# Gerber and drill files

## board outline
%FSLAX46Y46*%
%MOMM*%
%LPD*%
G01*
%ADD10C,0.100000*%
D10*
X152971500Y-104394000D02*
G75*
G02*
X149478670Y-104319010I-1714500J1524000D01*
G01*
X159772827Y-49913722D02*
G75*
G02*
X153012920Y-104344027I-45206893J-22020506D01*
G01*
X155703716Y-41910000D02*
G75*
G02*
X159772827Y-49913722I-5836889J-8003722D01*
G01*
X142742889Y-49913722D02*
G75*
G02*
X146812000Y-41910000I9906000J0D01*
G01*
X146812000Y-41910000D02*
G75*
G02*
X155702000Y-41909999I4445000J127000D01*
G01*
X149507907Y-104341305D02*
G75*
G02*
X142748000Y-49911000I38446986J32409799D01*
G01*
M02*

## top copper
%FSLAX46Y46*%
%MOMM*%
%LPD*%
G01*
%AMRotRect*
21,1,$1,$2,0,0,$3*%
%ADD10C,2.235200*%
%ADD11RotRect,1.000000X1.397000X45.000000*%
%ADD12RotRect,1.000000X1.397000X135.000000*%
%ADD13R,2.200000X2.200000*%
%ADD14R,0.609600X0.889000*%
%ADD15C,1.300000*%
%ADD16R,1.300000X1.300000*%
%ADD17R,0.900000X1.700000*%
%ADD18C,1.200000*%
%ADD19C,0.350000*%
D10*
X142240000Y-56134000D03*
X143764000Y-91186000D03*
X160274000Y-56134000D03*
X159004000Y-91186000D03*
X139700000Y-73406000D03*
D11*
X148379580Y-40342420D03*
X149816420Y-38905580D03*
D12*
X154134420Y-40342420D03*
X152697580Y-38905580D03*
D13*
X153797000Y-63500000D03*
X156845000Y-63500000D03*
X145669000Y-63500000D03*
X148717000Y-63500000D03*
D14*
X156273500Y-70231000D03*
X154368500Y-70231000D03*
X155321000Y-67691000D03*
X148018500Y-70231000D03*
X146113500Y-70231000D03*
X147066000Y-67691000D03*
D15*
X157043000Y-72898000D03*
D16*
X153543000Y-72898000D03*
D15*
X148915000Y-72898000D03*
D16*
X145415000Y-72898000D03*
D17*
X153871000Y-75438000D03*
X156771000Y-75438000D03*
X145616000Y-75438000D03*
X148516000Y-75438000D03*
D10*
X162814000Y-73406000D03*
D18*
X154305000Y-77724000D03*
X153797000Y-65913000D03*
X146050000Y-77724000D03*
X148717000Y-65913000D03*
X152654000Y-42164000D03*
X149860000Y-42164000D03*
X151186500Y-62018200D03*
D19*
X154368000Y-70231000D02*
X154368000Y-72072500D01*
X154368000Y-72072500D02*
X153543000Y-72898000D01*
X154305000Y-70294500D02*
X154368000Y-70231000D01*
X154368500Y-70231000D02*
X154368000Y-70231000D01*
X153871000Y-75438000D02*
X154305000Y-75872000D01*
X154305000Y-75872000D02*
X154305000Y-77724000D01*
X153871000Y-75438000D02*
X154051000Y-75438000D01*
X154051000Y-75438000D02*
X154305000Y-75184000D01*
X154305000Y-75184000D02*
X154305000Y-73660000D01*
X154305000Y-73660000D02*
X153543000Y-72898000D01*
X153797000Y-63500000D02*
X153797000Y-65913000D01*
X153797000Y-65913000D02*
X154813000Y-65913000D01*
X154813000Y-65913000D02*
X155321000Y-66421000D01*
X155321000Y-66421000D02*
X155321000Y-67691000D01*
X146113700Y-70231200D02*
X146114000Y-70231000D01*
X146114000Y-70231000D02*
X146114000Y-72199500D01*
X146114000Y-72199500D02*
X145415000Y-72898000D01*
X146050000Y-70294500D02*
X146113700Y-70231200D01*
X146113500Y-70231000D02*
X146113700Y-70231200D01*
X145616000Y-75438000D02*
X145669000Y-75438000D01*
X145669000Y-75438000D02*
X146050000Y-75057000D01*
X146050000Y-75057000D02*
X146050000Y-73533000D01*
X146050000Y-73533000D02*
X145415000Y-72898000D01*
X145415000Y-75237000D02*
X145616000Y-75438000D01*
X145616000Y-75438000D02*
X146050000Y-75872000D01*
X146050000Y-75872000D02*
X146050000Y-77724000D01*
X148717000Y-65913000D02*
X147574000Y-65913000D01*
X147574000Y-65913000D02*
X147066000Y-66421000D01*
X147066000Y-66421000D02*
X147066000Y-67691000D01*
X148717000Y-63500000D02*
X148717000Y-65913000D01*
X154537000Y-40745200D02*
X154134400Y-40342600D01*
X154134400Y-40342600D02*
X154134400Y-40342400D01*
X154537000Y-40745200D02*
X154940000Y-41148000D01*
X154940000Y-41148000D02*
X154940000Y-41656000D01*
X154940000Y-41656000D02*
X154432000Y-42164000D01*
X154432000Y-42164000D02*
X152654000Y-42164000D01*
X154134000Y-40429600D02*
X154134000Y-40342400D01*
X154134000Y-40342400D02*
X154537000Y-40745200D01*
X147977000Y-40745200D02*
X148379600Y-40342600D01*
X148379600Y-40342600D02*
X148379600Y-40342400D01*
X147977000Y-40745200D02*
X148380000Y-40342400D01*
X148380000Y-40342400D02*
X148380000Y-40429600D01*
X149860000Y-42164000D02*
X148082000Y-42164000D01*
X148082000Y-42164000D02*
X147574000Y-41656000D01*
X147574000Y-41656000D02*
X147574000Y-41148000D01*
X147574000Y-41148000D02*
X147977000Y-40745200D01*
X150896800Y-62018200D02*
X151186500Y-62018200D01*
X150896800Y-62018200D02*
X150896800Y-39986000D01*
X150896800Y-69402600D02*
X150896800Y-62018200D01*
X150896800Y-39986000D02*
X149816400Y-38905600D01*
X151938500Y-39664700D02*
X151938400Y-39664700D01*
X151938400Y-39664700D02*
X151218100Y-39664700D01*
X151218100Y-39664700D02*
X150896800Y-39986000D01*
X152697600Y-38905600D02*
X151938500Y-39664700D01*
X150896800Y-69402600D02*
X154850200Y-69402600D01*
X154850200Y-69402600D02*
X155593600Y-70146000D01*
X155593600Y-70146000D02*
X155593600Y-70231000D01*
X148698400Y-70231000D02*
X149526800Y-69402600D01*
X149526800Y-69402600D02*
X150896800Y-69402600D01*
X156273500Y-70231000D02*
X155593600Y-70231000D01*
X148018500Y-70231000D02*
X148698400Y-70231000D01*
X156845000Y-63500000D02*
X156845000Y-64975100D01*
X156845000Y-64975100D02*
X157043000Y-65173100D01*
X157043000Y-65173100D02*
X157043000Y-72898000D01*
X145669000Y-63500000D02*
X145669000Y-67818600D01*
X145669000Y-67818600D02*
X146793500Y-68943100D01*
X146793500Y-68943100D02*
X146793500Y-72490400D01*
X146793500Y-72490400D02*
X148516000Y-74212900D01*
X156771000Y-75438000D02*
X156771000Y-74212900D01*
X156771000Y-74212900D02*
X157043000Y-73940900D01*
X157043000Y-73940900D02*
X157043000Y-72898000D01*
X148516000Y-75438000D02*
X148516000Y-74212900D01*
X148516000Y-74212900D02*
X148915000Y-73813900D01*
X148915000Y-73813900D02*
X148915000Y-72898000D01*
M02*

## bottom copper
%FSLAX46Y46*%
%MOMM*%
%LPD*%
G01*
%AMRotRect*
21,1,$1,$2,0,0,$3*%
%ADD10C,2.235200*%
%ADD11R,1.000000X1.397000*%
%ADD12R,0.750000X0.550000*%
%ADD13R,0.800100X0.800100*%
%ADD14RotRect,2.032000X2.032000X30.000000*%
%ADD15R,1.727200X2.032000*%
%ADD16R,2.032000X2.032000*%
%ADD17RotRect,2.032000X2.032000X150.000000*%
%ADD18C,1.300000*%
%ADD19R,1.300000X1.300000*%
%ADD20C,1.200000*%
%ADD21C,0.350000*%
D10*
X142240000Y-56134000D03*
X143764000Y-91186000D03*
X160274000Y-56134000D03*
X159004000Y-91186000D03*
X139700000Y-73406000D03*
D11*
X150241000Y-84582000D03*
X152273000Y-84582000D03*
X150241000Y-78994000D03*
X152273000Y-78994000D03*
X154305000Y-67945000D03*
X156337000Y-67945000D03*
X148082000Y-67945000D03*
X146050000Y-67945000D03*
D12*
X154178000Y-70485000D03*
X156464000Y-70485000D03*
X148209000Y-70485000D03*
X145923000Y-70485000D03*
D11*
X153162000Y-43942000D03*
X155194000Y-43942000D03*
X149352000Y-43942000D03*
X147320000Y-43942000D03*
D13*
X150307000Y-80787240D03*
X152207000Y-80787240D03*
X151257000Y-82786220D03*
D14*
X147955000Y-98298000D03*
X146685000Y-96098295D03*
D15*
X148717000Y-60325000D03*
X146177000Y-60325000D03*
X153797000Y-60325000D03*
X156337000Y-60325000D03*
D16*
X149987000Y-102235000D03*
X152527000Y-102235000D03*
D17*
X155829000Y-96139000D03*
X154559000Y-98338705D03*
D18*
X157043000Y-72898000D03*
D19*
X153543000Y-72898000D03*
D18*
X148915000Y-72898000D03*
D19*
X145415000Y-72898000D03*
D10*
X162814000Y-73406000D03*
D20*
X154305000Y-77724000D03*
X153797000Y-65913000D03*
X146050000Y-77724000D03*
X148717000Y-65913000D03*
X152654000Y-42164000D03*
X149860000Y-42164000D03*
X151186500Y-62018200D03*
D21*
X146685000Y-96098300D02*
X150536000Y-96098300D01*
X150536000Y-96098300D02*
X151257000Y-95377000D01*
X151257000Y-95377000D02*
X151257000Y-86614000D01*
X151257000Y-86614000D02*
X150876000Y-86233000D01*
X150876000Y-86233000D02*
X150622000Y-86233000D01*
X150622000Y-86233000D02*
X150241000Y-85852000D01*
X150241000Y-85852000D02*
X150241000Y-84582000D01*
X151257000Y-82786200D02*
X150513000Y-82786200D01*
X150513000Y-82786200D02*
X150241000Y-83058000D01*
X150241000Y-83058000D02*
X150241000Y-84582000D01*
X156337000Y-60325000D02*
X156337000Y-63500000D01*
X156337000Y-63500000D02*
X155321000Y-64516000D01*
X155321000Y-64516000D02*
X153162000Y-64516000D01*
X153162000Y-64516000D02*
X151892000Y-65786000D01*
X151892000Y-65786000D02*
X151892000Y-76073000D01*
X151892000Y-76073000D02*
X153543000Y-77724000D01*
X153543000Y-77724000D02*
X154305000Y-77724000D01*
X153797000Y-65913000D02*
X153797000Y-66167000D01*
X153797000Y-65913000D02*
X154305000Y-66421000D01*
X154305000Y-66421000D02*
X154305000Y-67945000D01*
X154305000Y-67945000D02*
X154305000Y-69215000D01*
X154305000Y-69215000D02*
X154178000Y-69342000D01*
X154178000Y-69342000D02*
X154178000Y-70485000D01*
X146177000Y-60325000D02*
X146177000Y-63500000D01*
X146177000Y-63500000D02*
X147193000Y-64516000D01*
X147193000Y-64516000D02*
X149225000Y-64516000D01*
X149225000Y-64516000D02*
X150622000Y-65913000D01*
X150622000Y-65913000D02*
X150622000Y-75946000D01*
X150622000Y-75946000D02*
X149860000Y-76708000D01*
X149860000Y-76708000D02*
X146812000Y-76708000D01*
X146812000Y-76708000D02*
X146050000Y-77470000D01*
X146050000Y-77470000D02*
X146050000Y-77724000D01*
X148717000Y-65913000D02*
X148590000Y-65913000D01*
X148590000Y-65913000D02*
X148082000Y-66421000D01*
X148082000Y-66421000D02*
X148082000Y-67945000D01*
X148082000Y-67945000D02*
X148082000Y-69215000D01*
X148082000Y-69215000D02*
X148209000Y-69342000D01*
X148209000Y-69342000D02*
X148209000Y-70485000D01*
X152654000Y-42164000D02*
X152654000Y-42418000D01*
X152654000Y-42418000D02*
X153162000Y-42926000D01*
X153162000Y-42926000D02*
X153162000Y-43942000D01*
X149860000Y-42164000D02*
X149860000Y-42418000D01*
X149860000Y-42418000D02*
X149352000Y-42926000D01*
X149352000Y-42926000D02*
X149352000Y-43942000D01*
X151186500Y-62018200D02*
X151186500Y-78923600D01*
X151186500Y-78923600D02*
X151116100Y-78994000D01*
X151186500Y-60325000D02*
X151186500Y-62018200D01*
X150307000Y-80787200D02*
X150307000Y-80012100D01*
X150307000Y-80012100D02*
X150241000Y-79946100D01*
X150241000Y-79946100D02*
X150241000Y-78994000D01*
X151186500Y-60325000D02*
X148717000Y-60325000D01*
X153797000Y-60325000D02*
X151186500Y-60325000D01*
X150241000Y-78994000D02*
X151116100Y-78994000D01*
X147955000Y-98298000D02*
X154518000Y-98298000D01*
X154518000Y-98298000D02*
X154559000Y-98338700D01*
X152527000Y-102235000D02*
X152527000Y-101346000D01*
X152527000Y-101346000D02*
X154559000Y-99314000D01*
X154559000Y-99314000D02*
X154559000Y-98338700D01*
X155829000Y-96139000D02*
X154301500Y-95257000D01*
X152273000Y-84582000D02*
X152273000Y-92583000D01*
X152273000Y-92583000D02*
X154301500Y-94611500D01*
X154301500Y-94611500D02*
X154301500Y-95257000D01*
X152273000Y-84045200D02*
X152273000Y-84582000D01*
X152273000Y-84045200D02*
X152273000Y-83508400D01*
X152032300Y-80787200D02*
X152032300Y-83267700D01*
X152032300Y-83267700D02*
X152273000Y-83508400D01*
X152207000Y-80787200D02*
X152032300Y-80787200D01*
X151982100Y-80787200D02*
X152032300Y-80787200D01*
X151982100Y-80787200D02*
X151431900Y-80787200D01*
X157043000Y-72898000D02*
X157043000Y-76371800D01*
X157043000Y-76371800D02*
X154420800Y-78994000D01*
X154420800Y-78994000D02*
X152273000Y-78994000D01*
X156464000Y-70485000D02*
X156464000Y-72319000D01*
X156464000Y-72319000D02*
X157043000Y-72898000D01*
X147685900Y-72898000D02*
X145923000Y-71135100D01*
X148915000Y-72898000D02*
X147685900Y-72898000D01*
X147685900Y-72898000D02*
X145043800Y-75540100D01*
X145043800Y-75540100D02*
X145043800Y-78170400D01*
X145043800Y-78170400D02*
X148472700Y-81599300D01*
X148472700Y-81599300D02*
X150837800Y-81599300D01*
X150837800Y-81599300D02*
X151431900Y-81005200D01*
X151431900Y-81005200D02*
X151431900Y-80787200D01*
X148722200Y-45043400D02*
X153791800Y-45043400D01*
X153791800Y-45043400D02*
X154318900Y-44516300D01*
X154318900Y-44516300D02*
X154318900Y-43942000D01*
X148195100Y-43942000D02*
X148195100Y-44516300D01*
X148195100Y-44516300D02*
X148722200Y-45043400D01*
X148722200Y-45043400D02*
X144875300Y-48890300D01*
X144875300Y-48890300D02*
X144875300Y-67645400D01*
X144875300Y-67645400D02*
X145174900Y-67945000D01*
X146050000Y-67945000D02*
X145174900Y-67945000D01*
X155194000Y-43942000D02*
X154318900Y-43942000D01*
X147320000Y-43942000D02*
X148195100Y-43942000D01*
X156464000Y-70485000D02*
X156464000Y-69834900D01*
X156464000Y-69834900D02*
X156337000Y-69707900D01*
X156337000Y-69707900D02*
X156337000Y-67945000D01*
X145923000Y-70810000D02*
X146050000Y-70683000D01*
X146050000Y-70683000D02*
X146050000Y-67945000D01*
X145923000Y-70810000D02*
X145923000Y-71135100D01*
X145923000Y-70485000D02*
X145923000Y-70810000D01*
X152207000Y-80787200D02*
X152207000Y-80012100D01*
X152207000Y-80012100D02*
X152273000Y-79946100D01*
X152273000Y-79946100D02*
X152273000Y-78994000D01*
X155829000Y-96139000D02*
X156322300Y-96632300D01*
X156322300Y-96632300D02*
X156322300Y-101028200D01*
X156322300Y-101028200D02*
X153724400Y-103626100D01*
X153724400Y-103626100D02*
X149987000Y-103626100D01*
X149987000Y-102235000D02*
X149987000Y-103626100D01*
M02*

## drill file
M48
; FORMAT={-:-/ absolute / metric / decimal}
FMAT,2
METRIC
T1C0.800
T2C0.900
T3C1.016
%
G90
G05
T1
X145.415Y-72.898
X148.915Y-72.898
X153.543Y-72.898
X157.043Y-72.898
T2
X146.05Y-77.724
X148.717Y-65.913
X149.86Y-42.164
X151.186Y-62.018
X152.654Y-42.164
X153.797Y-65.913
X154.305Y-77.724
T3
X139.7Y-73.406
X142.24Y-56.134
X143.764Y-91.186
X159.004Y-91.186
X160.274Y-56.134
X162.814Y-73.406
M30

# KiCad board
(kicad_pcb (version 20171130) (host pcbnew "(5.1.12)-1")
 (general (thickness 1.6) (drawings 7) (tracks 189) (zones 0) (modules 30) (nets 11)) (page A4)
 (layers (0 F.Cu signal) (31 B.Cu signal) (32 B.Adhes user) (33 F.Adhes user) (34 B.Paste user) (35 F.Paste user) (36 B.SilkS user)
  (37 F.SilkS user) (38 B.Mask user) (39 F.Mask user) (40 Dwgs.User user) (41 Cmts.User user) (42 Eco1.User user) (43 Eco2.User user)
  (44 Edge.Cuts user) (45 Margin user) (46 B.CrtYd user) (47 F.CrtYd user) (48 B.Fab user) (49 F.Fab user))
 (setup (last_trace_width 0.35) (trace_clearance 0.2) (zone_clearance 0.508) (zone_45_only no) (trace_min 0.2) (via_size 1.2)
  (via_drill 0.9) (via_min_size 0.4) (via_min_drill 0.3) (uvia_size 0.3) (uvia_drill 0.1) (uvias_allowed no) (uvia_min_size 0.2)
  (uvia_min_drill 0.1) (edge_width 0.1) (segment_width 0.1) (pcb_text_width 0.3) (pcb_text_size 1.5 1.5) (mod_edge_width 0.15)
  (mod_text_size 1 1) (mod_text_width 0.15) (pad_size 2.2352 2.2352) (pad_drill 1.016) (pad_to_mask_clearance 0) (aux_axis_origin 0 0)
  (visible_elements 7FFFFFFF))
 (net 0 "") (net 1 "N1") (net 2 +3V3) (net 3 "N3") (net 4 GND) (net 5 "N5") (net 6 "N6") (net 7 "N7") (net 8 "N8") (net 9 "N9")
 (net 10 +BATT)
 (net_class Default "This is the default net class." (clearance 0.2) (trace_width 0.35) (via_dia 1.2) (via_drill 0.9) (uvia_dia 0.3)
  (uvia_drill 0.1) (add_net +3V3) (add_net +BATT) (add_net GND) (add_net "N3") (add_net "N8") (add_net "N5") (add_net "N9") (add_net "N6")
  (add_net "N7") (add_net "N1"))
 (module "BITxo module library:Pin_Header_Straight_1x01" (layer F.Cu) (at 142.24 56.134)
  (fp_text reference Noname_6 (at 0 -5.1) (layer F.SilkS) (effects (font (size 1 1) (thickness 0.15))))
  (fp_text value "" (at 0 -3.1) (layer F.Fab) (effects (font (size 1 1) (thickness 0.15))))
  (pad 1 thru_hole circle (at 0 0) (size 2.2352 2.2352) (drill 1.016) (layers *.Cu *.Mask F.SilkS)))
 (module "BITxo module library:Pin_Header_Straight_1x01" (layer F.Cu) (at 143.764 91.186)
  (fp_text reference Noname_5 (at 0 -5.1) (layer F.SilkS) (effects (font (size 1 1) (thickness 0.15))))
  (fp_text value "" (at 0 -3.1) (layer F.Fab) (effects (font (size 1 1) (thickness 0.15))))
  (pad 1 thru_hole circle (at 0 0) (size 2.2352 2.2352) (drill 1.016) (layers *.Cu *.Mask F.SilkS)))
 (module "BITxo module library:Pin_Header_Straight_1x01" (layer F.Cu) (at 160.274 56.134)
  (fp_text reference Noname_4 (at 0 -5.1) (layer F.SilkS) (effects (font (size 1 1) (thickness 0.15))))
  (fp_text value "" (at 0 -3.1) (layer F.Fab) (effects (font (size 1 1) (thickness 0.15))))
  (pad 1 thru_hole circle (at 0 0) (size 2.2352 2.2352) (drill 1.016) (layers *.Cu *.Mask F.SilkS)))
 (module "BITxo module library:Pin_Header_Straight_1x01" (layer F.Cu) (at 159.004 91.186)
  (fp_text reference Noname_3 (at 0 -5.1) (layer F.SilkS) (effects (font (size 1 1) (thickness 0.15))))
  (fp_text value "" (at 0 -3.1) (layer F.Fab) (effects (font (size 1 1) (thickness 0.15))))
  (pad 1 thru_hole circle (at 0 0) (size 2.2352 2.2352) (drill 1.016) (layers *.Cu *.Mask F.SilkS)))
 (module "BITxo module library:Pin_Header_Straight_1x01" (layer F.Cu) (at 139.7 73.406)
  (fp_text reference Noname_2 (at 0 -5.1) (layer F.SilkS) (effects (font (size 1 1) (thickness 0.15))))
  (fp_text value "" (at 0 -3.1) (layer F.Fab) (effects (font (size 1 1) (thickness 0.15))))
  (pad 1 thru_hole circle (at 0 0) (size 2.2352 2.2352) (drill 1.016) (layers *.Cu *.Mask F.SilkS)))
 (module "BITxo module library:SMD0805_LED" (layer F.Cu) (at 149.098 39.624 45)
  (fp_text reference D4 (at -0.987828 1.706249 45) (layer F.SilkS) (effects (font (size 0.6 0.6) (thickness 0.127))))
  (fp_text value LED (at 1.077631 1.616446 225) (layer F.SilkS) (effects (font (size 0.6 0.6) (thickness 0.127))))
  (pad 1 smd rect (at -1.016 0 45) (size 1 1.397) (layers F.Cu F.Paste F.Mask) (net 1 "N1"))
  (pad 2 smd rect (at 1.016 0 45) (size 1 1.397) (layers F.Cu F.Paste F.Mask) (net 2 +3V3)))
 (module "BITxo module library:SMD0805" (layer B.Cu) (at 151.257 84.582)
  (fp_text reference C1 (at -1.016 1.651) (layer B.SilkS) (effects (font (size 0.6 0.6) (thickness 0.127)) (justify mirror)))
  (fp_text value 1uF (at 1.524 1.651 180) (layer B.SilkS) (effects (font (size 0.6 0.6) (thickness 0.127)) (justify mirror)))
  (pad 1 smd rect (at -1.016 0) (size 1 1.397) (layers B.Cu B.Paste B.Mask) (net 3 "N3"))
  (pad 2 smd rect (at 1.016 0) (size 1 1.397) (layers B.Cu B.Paste B.Mask) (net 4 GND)))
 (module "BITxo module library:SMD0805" (layer B.Cu) (at 151.257 78.994)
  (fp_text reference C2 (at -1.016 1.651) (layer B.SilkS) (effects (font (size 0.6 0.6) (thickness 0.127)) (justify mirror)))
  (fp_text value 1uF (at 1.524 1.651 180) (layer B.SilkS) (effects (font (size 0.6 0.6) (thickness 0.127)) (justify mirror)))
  (pad 1 smd rect (at -1.016 0) (size 1 1.397) (layers B.Cu B.Paste B.Mask) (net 2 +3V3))
  (pad 2 smd rect (at 1.016 0) (size 1 1.397) (layers B.Cu B.Paste B.Mask) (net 4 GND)))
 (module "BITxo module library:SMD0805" (layer B.Cu) (at 155.321 67.945)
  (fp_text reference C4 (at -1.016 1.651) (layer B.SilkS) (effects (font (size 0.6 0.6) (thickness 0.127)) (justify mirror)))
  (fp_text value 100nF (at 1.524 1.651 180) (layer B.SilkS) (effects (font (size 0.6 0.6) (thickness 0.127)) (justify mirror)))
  (pad 1 smd rect (at -1.016 0) (size 1 1.397) (layers B.Cu B.Paste B.Mask) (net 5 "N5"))
  (pad 2 smd rect (at 1.016 0) (size 1 1.397) (layers B.Cu B.Paste B.Mask) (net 4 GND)))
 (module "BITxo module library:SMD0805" (layer B.Cu) (at 147.066 67.945 180)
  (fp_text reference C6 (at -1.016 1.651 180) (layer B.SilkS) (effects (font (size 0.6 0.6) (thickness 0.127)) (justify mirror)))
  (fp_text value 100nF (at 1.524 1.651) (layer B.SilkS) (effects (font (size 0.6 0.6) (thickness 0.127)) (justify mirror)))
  (pad 1 smd rect (at -1.016 0 180) (size 1 1.397) (layers B.Cu B.Paste B.Mask) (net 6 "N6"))
  (pad 2 smd rect (at 1.016 0 180) (size 1 1.397) (layers B.Cu B.Paste B.Mask) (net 4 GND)))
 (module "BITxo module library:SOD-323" (layer B.Cu) (at 155.321 70.485)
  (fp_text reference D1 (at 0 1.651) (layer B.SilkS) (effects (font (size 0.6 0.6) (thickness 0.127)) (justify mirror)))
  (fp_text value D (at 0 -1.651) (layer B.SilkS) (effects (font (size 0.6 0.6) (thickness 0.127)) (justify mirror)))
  (pad 1 smd rect (at -1.143 0) (size 0.75 0.55) (layers B.Cu B.Paste B.Mask) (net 5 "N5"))
  (pad 2 smd rect (at 1.143 0) (size 0.75 0.55) (layers B.Cu B.Paste B.Mask) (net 4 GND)))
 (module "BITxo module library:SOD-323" (layer B.Cu) (at 147.066 70.485 180)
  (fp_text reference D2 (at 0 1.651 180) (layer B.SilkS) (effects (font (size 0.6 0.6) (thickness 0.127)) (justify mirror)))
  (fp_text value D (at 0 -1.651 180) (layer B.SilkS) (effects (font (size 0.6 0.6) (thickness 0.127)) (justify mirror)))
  (pad 1 smd rect (at -1.143 0 180) (size 0.75 0.55) (layers B.Cu B.Paste B.Mask) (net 6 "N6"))
  (pad 2 smd rect (at 1.143 0 180) (size 0.75 0.55) (layers B.Cu B.Paste B.Mask) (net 4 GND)))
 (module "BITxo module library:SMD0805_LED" (layer F.Cu) (at 153.416 39.624 135)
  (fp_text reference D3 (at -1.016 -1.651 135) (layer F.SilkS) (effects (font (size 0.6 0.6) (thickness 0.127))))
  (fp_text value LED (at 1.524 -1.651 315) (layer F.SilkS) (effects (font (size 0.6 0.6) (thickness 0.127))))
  (pad 1 smd rect (at -1.016 0 135) (size 1 1.397) (layers F.Cu F.Paste F.Mask) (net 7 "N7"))
  (pad 2 smd rect (at 1.016 0 135) (size 1 1.397) (layers F.Cu F.Paste F.Mask) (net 2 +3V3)))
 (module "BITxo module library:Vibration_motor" (layer F.Cu) (at 155.321 63.5)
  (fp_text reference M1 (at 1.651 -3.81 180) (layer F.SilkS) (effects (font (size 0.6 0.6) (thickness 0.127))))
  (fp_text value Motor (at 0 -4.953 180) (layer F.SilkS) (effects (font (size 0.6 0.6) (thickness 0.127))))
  (pad 1 smd rect (at -1.524 0) (size 2.2 2.2) (layers F.Cu F.Paste F.Mask) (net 5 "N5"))
  (pad 2 smd rect (at 1.524 0) (size 2.2 2.2) (layers F.Cu F.Paste F.Mask) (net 4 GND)))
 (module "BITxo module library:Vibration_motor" (layer F.Cu) (at 147.193 63.5)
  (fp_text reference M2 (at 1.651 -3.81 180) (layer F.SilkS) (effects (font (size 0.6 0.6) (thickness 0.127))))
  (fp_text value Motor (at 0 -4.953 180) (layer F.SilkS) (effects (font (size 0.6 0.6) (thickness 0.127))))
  (pad 1 smd rect (at -1.524 0) (size 2.2 2.2) (layers F.Cu F.Paste F.Mask) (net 4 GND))
  (pad 2 smd rect (at 1.524 0) (size 2.2 2.2) (layers F.Cu F.Paste F.Mask) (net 6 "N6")))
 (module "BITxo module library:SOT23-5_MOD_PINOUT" (layer F.Cu) (at 155.321 68.961)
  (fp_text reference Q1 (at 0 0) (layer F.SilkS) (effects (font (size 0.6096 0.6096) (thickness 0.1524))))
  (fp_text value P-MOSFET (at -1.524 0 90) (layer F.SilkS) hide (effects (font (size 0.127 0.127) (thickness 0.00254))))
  (pad 3 smd rect (at 0.9525 1.27) (size 0.6096 0.889) (layers F.Cu F.Paste F.Mask) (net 2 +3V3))
  (pad 2 smd rect (at -0.9525 1.27) (size 0.6096 0.889) (layers F.Cu F.Paste F.Mask) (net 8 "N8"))
  (pad 1 smd rect (at 0 -1.27) (size 0.6096 0.889) (layers F.Cu F.Paste F.Mask) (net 5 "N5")))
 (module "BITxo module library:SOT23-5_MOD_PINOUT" (layer F.Cu) (at 147.066 68.961)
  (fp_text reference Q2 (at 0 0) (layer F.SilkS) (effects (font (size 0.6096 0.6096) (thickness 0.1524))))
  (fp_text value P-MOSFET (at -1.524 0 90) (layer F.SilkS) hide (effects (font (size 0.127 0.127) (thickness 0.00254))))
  (pad 3 smd rect (at 0.9525 1.27) (size 0.6096 0.889) (layers F.Cu F.Paste F.Mask) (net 2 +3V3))
  (pad 2 smd rect (at -0.9525 1.27) (size 0.6096 0.889) (layers F.Cu F.Paste F.Mask) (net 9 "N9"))
  (pad 1 smd rect (at 0 -1.27) (size 0.6096 0.889) (layers F.Cu F.Paste F.Mask) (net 6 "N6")))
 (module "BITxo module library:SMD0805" (layer B.Cu) (at 154.178 43.942)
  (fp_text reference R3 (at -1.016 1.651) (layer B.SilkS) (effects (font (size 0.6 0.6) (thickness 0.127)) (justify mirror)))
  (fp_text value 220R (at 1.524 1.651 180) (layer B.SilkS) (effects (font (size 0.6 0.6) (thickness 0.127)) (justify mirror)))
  (pad 1 smd rect (at -1.016 0) (size 1 1.397) (layers B.Cu B.Paste B.Mask) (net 7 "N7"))
  (pad 2 smd rect (at 1.016 0) (size 1 1.397) (layers B.Cu B.Paste B.Mask) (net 4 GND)))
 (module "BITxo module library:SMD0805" (layer B.Cu) (at 148.336 43.942 180)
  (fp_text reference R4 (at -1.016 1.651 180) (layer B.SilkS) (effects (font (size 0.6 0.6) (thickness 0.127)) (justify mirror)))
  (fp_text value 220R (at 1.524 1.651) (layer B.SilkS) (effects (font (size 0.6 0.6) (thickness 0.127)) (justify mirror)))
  (pad 1 smd rect (at -1.016 0 180) (size 1 1.397) (layers B.Cu B.Paste B.Mask) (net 1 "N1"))
  (pad 2 smd rect (at 1.016 0 180) (size 1 1.397) (layers B.Cu B.Paste B.Mask) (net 4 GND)))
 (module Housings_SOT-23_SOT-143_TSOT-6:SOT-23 (layer B.Cu) (at 151.257 81.788)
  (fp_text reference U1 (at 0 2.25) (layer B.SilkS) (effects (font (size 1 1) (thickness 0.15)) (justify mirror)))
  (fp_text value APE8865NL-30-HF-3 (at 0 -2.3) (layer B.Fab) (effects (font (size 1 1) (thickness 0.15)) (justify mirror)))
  (pad 1 smd rect (at -0.95 -1.00076) (size 0.8001 0.8001) (layers B.Cu B.Paste B.Mask) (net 2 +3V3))
  (pad 2 smd rect (at 0.95 -1.00076) (size 0.8001 0.8001) (layers B.Cu B.Paste B.Mask) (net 4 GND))
  (pad 3 smd rect (at 0 0.99822) (size 0.8001 0.8001) (layers B.Cu B.Paste B.Mask) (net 3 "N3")))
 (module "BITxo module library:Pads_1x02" (layer B.Cu) (at 147.955 98.298 30)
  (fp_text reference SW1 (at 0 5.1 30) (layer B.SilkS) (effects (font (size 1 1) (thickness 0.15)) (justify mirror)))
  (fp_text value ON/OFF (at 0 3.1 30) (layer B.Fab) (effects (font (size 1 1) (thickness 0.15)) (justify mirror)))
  (pad 1 smd rect (at 0 0 30) (size 2.032 2.032) (layers B.Cu B.Paste B.Mask) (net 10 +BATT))
  (pad 2 smd rect (at 0 -2.54 30) (size 2.032 2.032) (layers B.Cu B.Paste B.Mask) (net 3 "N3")))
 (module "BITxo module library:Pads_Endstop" (layer B.Cu) (at 151.257 60.325 90)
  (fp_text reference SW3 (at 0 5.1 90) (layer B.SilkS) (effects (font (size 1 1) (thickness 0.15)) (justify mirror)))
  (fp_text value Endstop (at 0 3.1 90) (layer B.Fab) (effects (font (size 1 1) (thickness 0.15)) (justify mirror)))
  (pad 2 smd rect (at 0 -2.54 90) (size 2.032 1.7272) (layers B.Cu B.Paste B.Mask) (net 2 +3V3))
  (pad 3 smd rect (at 0 -5.08 90) (size 2.032 1.7272) (layers B.Cu B.Paste B.Mask) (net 9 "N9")))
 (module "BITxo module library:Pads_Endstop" (layer B.Cu) (at 151.257 60.325 270)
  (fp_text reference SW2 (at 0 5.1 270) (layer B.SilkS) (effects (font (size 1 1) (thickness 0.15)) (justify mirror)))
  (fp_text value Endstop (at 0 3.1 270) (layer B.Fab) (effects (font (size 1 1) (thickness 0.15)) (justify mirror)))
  (pad 2 smd rect (at 0 -2.54 270) (size 2.032 1.7272) (layers B.Cu B.Paste B.Mask) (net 2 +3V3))
  (pad 3 smd rect (at 0 -5.08 270) (size 2.032 1.7272) (layers B.Cu B.Paste B.Mask) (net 8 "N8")))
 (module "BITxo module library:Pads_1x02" (layer B.Cu) (at 149.987 102.235 270)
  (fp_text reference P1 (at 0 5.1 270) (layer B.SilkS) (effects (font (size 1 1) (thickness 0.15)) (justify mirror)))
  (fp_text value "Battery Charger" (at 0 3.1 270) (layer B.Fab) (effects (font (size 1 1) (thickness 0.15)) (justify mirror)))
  (pad 1 smd rect (at 0 0 270) (size 2.032 2.032) (layers B.Cu B.Paste B.Mask) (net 4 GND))
  (pad 2 smd rect (at 0 -2.54 270) (size 2.032 2.032) (layers B.Cu B.Paste B.Mask) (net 10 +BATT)))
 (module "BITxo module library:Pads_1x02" (layer B.Cu) (at 155.829 96.139 150)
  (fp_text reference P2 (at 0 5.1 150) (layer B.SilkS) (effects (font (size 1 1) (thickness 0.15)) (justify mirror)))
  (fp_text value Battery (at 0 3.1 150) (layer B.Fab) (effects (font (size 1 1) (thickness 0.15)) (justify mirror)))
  (pad 1 smd rect (at 0 0 150) (size 2.032 2.032) (layers B.Cu B.Paste B.Mask) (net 4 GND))
  (pad 2 smd rect (at 0 -2.54 150) (size 2.032 2.032) (layers B.Cu B.Paste B.Mask) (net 10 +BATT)))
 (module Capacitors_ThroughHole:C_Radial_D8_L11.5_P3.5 (layer F.Cu) (at 153.543 72.898)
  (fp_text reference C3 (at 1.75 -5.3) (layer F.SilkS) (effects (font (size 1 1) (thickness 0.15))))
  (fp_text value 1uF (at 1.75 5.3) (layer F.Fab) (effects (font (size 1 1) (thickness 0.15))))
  (pad 2 thru_hole circle (at 3.5 0) (size 1.3 1.3) (drill 0.8) (layers *.Cu *.Mask F.SilkS) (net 4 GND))
  (pad 1 thru_hole rect (at 0 0) (size 1.3 1.3) (drill 0.8) (layers *.Cu *.Mask F.SilkS) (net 8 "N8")))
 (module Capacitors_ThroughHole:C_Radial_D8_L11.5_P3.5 (layer F.Cu) (at 145.415 72.898)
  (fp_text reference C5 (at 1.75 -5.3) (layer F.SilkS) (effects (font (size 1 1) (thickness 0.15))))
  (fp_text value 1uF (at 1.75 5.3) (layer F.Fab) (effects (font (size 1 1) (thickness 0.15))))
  (pad 2 thru_hole circle (at 3.5 0) (size 1.3 1.3) (drill 0.8) (layers *.Cu *.Mask F.SilkS) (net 4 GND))
  (pad 1 thru_hole rect (at 0 0) (size 1.3 1.3) (drill 0.8) (layers *.Cu *.Mask F.SilkS) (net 9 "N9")))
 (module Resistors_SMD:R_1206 (layer F.Cu) (at 155.321 75.438)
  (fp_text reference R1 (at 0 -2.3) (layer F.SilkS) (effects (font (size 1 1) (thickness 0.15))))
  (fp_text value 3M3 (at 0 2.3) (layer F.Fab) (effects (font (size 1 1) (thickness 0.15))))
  (pad 1 smd rect (at -1.45 0) (size 0.9 1.7) (layers F.Cu F.Paste F.Mask) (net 8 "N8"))
  (pad 2 smd rect (at 1.45 0) (size 0.9 1.7) (layers F.Cu F.Paste F.Mask) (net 4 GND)))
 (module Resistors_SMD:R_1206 (layer F.Cu) (at 147.066 75.438)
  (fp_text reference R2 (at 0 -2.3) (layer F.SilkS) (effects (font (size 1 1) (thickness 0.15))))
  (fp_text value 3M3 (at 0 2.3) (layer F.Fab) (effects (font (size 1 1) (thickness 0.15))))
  (pad 1 smd rect (at -1.45 0) (size 0.9 1.7) (layers F.Cu F.Paste F.Mask) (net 9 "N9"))
  (pad 2 smd rect (at 1.45 0) (size 0.9 1.7) (layers F.Cu F.Paste F.Mask) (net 4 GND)))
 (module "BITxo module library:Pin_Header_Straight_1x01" (layer F.Cu) (at 162.814 73.406)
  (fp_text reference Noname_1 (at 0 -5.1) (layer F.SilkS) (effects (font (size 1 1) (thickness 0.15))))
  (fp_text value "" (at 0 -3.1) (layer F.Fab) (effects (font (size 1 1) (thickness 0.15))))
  (pad 1 thru_hole circle (at 0 0) (size 2.2352 2.2352) (drill 1.016) (layers *.Cu *.Mask F.SilkS)))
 (gr_arc (start 151.257 102.87) (end 152.9715 104.394) (angle 99.19279552) (layer Edge.Cuts) (width 0.1))
 (gr_arc (start 114.565934 71.934228) (end 153.01292 104.344027) (angle -66.10095577) (layer Edge.Cuts) (width 0.1))
 (gr_arc (start 149.866827 49.913722) (end 159.772827 49.913722) (angle -53.8977836) (layer Edge.Cuts) (width 0.1))
 (gr_arc (start 152.648889 49.913722) (end 142.742889 49.913722) (angle 53.8977836) (layer Edge.Cuts) (width 0.1))
 (gr_arc (start 151.257 41.783) (end 146.812 41.91) (angle 183.2731416) (layer Edge.Cuts) (width 0.1))
 (gr_arc (start 187.954893 71.931506) (end 149.507907 104.341305) (angle 66.10095577) (layer Edge.Cuts) (width 0.1))
 (segment (start 146.685 96.0983) (end 150.536 96.0983) (width 0.35) (layer B.Cu) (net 3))
 (segment (start 150.536 96.0983) (end 151.257 95.377) (width 0.35) (layer B.Cu) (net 3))
 (segment (start 151.257 95.377) (end 151.257 86.614) (width 0.35) (layer B.Cu) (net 3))
 (segment (start 151.257 86.614) (end 150.876 86.233) (width 0.35) (layer B.Cu) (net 3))
 (segment (start 150.876 86.233) (end 150.622 86.233) (width 0.35) (layer B.Cu) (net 3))
 (segment (start 150.622 86.233) (end 150.241 85.852) (width 0.35) (layer B.Cu) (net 3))
 (segment (start 150.241 85.852) (end 150.241 84.582) (width 0.35) (layer B.Cu) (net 3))
 (segment (start 151.257 82.7862) (end 150.513 82.7862) (width 0.35) (layer B.Cu) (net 3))
 (segment (start 150.513 82.7862) (end 150.241 83.058) (width 0.35) (layer B.Cu) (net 3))
 (segment (start 150.241 83.058) (end 150.241 84.582) (width 0.35) (layer B.Cu) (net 3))
 (segment (start 154.368 70.231) (end 154.368 72.0725) (width 0.35) (layer F.Cu) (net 8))
 (segment (start 154.368 72.0725) (end 153.543 72.898) (width 0.35) (layer F.Cu) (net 8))
 (segment (start 154.305 70.2945) (end 154.368 70.231) (width 0.35) (layer F.Cu) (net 8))
 (segment (start 154.3685 70.231) (end 154.368 70.231) (width 0.35) (layer F.Cu) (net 8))
 (segment (start 153.871 75.438) (end 154.305 75.872) (width 0.35) (layer F.Cu) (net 8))
 (segment (start 154.305 75.872) (end 154.305 77.724) (width 0.35) (layer F.Cu) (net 8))
 (segment (start 156.337 60.325) (end 156.337 63.5) (width 0.35) (layer B.Cu) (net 8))
 (segment (start 156.337 63.5) (end 155.321 64.516) (width 0.35) (layer B.Cu) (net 8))
 (segment (start 155.321 64.516) (end 153.162 64.516) (width 0.35) (layer B.Cu) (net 8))
 (segment (start 153.162 64.516) (end 151.892 65.786) (width 0.35) (layer B.Cu) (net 8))
 (segment (start 151.892 65.786) (end 151.892 76.073) (width 0.35) (layer B.Cu) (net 8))
 (segment (start 151.892 76.073) (end 153.543 77.724) (width 0.35) (layer B.Cu) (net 8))
 (segment (start 153.543 77.724) (end 154.305 77.724) (width 0.35) (layer B.Cu) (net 8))
 (segment (start 153.871 75.438) (end 154.051 75.438) (width 0.35) (layer F.Cu) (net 8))
 (segment (start 154.051 75.438) (end 154.305 75.184) (width 0.35) (layer F.Cu) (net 8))
 (segment (start 154.305 75.184) (end 154.305 73.66) (width 0.35) (layer F.Cu) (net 8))
 (segment (start 154.305 73.66) (end 153.543 72.898) (width 0.35) (layer F.Cu) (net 8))
 (via (at 154.305 77.724) (size 1.2) (layers F.Cu B.Cu) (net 8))
 (segment (start 153.797 65.913) (end 153.797 66.167) (width 0.35) (layer B.Cu) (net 5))
 (segment (start 153.797 63.5) (end 153.797 65.913) (width 0.35) (layer F.Cu) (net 5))
 (segment (start 153.797 65.913) (end 154.813 65.913) (width 0.35) (layer F.Cu) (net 5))
 (segment (start 154.813 65.913) (end 155.321 66.421) (width 0.35) (layer F.Cu) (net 5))
 (segment (start 155.321 66.421) (end 155.321 67.691) (width 0.35) (layer F.Cu) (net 5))
 (segment (start 153.797 65.913) (end 154.305 66.421) (width 0.35) (layer B.Cu) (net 5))
 (segment (start 154.305 66.421) (end 154.305 67.945) (width 0.35) (layer B.Cu) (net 5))
 (segment (start 154.305 67.945) (end 154.305 69.215) (width 0.35) (layer B.Cu) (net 5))
 (segment (start 154.305 69.215) (end 154.178 69.342) (width 0.35) (layer B.Cu) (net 5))
 (segment (start 154.178 69.342) (end 154.178 70.485) (width 0.35) (layer B.Cu) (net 5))
 (via (at 153.797 65.913) (size 1.2) (layers F.Cu B.Cu) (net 5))
 (segment (start 146.1137 70.2312) (end 146.114 70.231) (width 0.35) (layer F.Cu) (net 9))
 (segment (start 146.114 70.231) (end 146.114 72.1995) (width 0.35) (layer F.Cu) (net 9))
 (segment (start 146.114 72.1995) (end 145.415 72.898) (width 0.35) (layer F.Cu) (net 9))
 (segment (start 146.05 70.2945) (end 146.1137 70.2312) (width 0.35) (layer F.Cu) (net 9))
 (segment (start 146.1135 70.231) (end 146.1137 70.2312) (width 0.35) (layer F.Cu) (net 9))
 (segment (start 145.616 75.438) (end 145.669 75.438) (width 0.35) (layer F.Cu) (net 9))
 (segment (start 145.669 75.438) (end 146.05 75.057) (width 0.35) (layer F.Cu) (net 9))
 (segment (start 146.05 75.057) (end 146.05 73.533) (width 0.35) (layer F.Cu) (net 9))
 (segment (start 146.05 73.533) (end 145.415 72.898) (width 0.35) (layer F.Cu) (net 9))
 (segment (start 145.415 75.237) (end 145.616 75.438) (width 0.35) (layer F.Cu) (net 9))
 (segment (start 145.616 75.438) (end 146.05 75.872) (width 0.35) (layer F.Cu) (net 9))
 (segment (start 146.05 75.872) (end 146.05 77.724) (width 0.35) (layer F.Cu) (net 9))
 (segment (start 146.177 60.325) (end 146.177 63.5) (width 0.35) (layer B.Cu) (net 9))
 (segment (start 146.177 63.5) (end 147.193 64.516) (width 0.35) (layer B.Cu) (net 9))
 (segment (start 147.193 64.516) (end 149.225 64.516) (width 0.35) (layer B.Cu) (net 9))
 (segment (start 149.225 64.516) (end 150.622 65.913) (width 0.35) (layer B.Cu) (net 9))
 (segment (start 150.622 65.913) (end 150.622 75.946) (width 0.35) (layer B.Cu) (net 9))
 (segment (start 150.622 75.946) (end 149.86 76.708) (width 0.35) (layer B.Cu) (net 9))
 (segment (start 149.86 76.708) (end 146.812 76.708) (width 0.35) (layer B.Cu) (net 9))
 (segment (start 146.812 76.708) (end 146.05 77.47) (width 0.35) (layer B.Cu) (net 9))
 (segment (start 146.05 77.47) (end 146.05 77.724) (width 0.35) (layer B.Cu) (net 9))
 (via (at 146.05 77.724) (size 1.2) (layers F.Cu B.Cu) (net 9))
 (segment (start 148.717 65.913) (end 147.574 65.913) (width 0.35) (layer F.Cu) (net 6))
 (segment (start 147.574 65.913) (end 147.066 66.421) (width 0.35) (layer F.Cu) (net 6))
 (segment (start 147.066 66.421) (end 147.066 67.691) (width 0.35) (layer F.Cu) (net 6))
 (segment (start 148.717 63.5) (end 148.717 65.913) (width 0.35) (layer F.Cu) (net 6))
 (segment (start 148.717 65.913) (end 148.59 65.913) (width 0.35) (layer B.Cu) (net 6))
 (segment (start 148.59 65.913) (end 148.082 66.421) (width 0.35) (layer B.Cu) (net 6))
 (segment (start 148.082 66.421) (end 148.082 67.945) (width 0.35) (layer B.Cu) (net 6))
 (segment (start 148.082 67.945) (end 148.082 69.215) (width 0.35) (layer B.Cu) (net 6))
 (segment (start 148.082 69.215) (end 148.209 69.342) (width 0.35) (layer B.Cu) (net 6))
 (segment (start 148.209 69.342) (end 148.209 70.485) (width 0.35) (layer B.Cu) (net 6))
 (via (at 148.717 65.913) (size 1.2) (layers F.Cu B.Cu) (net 6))
 (segment (start 154.537 40.7452) (end 154.1344 40.3426) (width 0.35) (layer F.Cu) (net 7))
 (segment (start 154.1344 40.3426) (end 154.1344 40.3424) (width 0.35) (layer F.Cu) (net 7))
 (segment (start 154.537 40.7452) (end 154.94 41.148) (width 0.35) (layer F.Cu) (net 7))
 (segment (start 154.94 41.148) (end 154.94 41.656) (width 0.35) (layer F.Cu) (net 7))
 (segment (start 154.94 41.656) (end 154.432 42.164) (width 0.35) (layer F.Cu) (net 7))
 (segment (start 154.432 42.164) (end 152.654 42.164) (width 0.35) (layer F.Cu) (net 7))
 (segment (start 154.134 40.4296) (end 154.134 40.3424) (width 0.35) (layer F.Cu) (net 7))
 (segment (start 154.134 40.3424) (end 154.537 40.7452) (width 0.35) (layer F.Cu) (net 7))
 (segment (start 152.654 42.164) (end 152.654 42.418) (width 0.35) (layer B.Cu) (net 7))
 (segment (start 152.654 42.418) (end 153.162 42.926) (width 0.35) (layer B.Cu) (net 7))
 (segment (start 153.162 42.926) (end 153.162 43.942) (width 0.35) (layer B.Cu) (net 7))
 (via (at 152.654 42.164) (size 1.2) (layers F.Cu B.Cu) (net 7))
 (segment (start 147.977 40.7452) (end 148.3796 40.3426) (width 0.35) (layer F.Cu) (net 1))
 (segment (start 148.3796 40.3426) (end 148.3796 40.3424) (width 0.35) (layer F.Cu) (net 1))
 (segment (start 147.977 40.7452) (end 148.38 40.3424) (width 0.35) (layer F.Cu) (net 1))
 (segment (start 148.38 40.3424) (end 148.38 40.4296) (width 0.35) (layer F.Cu) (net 1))
 (segment (start 149.86 42.164) (end 148.082 42.164) (width 0.35) (layer F.Cu) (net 1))
 (segment (start 148.082 42.164) (end 147.574 41.656) (width 0.35) (layer F.Cu) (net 1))
 (segment (start 147.574 41.656) (end 147.574 41.148) (width 0.35) (layer F.Cu) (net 1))
 (segment (start 147.574 41.148) (end 147.977 40.7452) (width 0.35) (layer F.Cu) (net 1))
 (segment (start 149.86 42.164) (end 149.86 42.418) (width 0.35) (layer B.Cu) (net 1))
 (segment (start 149.86 42.418) (end 149.352 42.926) (width 0.35) (layer B.Cu) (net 1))
 (segment (start 149.352 42.926) (end 149.352 43.942) (width 0.35) (layer B.Cu) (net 1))
 (via (at 149.86 42.164) (size 1.2) (layers F.Cu B.Cu) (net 1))
 (segment (start 150.8968 62.0182) (end 151.1865 62.0182) (width 0.35) (layer F.Cu) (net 2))
 (segment (start 150.8968 62.0182) (end 150.8968 39.986) (width 0.35) (layer F.Cu) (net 2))
 (segment (start 150.8968 69.4026) (end 150.8968 62.0182) (width 0.35) (layer F.Cu) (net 2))
 (segment (start 151.1865 62.0182) (end 151.1865 78.9236) (width 0.35) (layer B.Cu) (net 2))
 (segment (start 151.1865 78.9236) (end 151.1161 78.994) (width 0.35) (layer B.Cu) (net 2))
 (segment (start 151.1865 60.325) (end 151.1865 62.0182) (width 0.35) (layer B.Cu) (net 2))
 (segment (start 150.8968 39.986) (end 149.8164 38.9056) (width 0.35) (layer F.Cu) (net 2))
 (segment (start 151.9385 39.6647) (end 151.9384 39.6647) (width 0.35) (layer F.Cu) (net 2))
 (segment (start 151.9384 39.6647) (end 151.2181 39.6647) (width 0.35) (layer F.Cu) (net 2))
 (segment (start 151.2181 39.6647) (end 150.8968 39.986) (width 0.35) (layer F.Cu) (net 2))
 (segment (start 152.6976 38.9056) (end 151.9385 39.6647) (width 0.35) (layer F.Cu) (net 2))
 (segment (start 150.8968 69.4026) (end 154.8502 69.4026) (width 0.35) (layer F.Cu) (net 2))
 (segment (start 154.8502 69.4026) (end 155.5936 70.146) (width 0.35) (layer F.Cu) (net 2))
 (segment (start 155.5936 70.146) (end 155.5936 70.231) (width 0.35) (layer F.Cu) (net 2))
 (segment (start 148.6984 70.231) (end 149.5268 69.4026) (width 0.35) (layer F.Cu) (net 2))
 (segment (start 149.5268 69.4026) (end 150.8968 69.4026) (width 0.35) (layer F.Cu) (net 2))
 (segment (start 156.2735 70.231) (end 155.5936 70.231) (width 0.35) (layer F.Cu) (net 2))
 (segment (start 148.0185 70.231) (end 148.6984 70.231) (width 0.35) (layer F.Cu) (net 2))
 (segment (start 150.307 80.7872) (end 150.307 80.0121) (width 0.35) (layer B.Cu) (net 2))
 (segment (start 150.307 80.0121) (end 150.241 79.9461) (width 0.35) (layer B.Cu) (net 2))
 (segment (start 150.241 79.9461) (end 150.241 78.994) (width 0.35) (layer B.Cu) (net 2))
 (segment (start 151.1865 60.325) (end 148.717 60.325) (width 0.35) (layer B.Cu) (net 2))
 (segment (start 153.797 60.325) (end 151.1865 60.325) (width 0.35) (layer B.Cu) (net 2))
 (segment (start 150.241 78.994) (end 151.1161 78.994) (width 0.35) (layer B.Cu) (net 2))
 (via (at 151.1865 62.0182) (size 1.2) (layers F.Cu B.Cu) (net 2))
 (segment (start 147.955 98.298) (end 154.518 98.298) (width 0.35) (layer B.Cu) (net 10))
 (segment (start 154.518 98.298) (end 154.559 98.3387) (width 0.35) (layer B.Cu) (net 10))
 (segment (start 152.527 102.235) (end 152.527 101.346) (width 0.35) (layer B.Cu) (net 10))
 (segment (start 152.527 101.346) (end 154.559 99.314) (width 0.35) (layer B.Cu) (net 10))
 (segment (start 154.559 99.314) (end 154.559 98.3387) (width 0.35) (layer B.Cu) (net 10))
 (segment (start 155.829 96.139) (end 154.3015 95.257) (width 0.35) (layer B.Cu) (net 4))
 (segment (start 152.273 84.582) (end 152.273 92.583) (width 0.35) (layer B.Cu) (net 4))
 (segment (start 152.273 92.583) (end 154.3015 94.6115) (width 0.35) (layer B.Cu) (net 4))
 (segment (start 154.3015 94.6115) (end 154.3015 95.257) (width 0.35) (layer B.Cu) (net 4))
 (segment (start 152.273 84.0452) (end 152.273 84.582) (width 0.35) (layer B.Cu) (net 4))
 (segment (start 152.273 84.0452) (end 152.273 83.5084) (width 0.35) (layer B.Cu) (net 4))
 (segment (start 152.0323 80.7872) (end 152.0323 83.2677) (width 0.35) (layer B.Cu) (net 4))
 (segment (start 152.0323 83.2677) (end 152.273 83.5084) (width 0.35) (layer B.Cu) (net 4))
 (segment (start 152.207 80.7872) (end 152.0323 80.7872) (width 0.35) (layer B.Cu) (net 4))
 (segment (start 151.9821 80.7872) (end 152.0323 80.7872) (width 0.35) (layer B.Cu) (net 4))
 (segment (start 151.9821 80.7872) (end 151.4319 80.7872) (width 0.35) (layer B.Cu) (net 4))
 (segment (start 157.043 72.898) (end 157.043 76.3718) (width 0.35) (layer B.Cu) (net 4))
 (segment (start 157.043 76.3718) (end 154.4208 78.994) (width 0.35) (layer B.Cu) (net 4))
 (segment (start 154.4208 78.994) (end 152.273 78.994) (width 0.35) (layer B.Cu) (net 4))
 (segment (start 156.464 70.485) (end 156.464 72.319) (width 0.35) (layer B.Cu) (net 4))
 (segment (start 156.464 72.319) (end 157.043 72.898) (width 0.35) (layer B.Cu) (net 4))
 (segment (start 147.6859 72.898) (end 145.923 71.1351) (width 0.35) (layer B.Cu) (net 4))
 (segment (start 148.915 72.898) (end 147.6859 72.898) (width 0.35) (layer B.Cu) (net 4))
 (segment (start 147.6859 72.898) (end 145.0438 75.5401) (width 0.35) (layer B.Cu) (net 4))
 (segment (start 145.0438 75.5401) (end 145.0438 78.1704) (width 0.35) (layer B.Cu) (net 4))
 (segment (start 145.0438 78.1704) (end 148.4727 81.5993) (width 0.35) (layer B.Cu) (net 4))
 (segment (start 148.4727 81.5993) (end 150.8378 81.5993) (width 0.35) (layer B.Cu) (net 4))
 (segment (start 150.8378 81.5993) (end 151.4319 81.0052) (width 0.35) (layer B.Cu) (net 4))
 (segment (start 151.4319 81.0052) (end 151.4319 80.7872) (width 0.35) (layer B.Cu) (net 4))
 (segment (start 148.7222 45.0434) (end 153.7918 45.0434) (width 0.35) (layer B.Cu) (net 4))
 (segment (start 153.7918 45.0434) (end 154.3189 44.5163) (width 0.35) (layer B.Cu) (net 4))
 (segment (start 154.3189 44.5163) (end 154.3189 43.942) (width 0.35) (layer B.Cu) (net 4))
 (segment (start 148.1951 43.942) (end 148.1951 44.5163) (width 0.35) (layer B.Cu) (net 4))
 (segment (start 148.1951 44.5163) (end 148.7222 45.0434) (width 0.35) (layer B.Cu) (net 4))
 (segment (start 148.7222 45.0434) (end 144.8753 48.8903) (width 0.35) (layer B.Cu) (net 4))
 (segment (start 144.8753 48.8903) (end 144.8753 67.6454) (width 0.35) (layer B.Cu) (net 4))
 (segment (start 144.8753 67.6454) (end 145.1749 67.945) (width 0.35) (layer B.Cu) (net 4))
 (segment (start 146.05 67.945) (end 145.1749 67.945) (width 0.35) (layer B.Cu) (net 4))
 (segment (start 155.194 43.942) (end 154.3189 43.942) (width 0.35) (layer B.Cu) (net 4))
 (segment (start 147.32 43.942) (end 148.1951 43.942) (width 0.35) (layer B.Cu) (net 4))
 (segment (start 156.464 70.485) (end 156.464 69.8349) (width 0.35) (layer B.Cu) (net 4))
 (segment (start 156.464 69.8349) (end 156.337 69.7079) (width 0.35) (layer B.Cu) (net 4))
 (segment (start 156.337 69.7079) (end 156.337 67.945) (width 0.35) (layer B.Cu) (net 4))
 (segment (start 145.923 70.81) (end 146.05 70.683) (width 0.35) (layer B.Cu) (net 4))
 (segment (start 146.05 70.683) (end 146.05 67.945) (width 0.35) (layer B.Cu) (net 4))
 (segment (start 145.923 70.81) (end 145.923 71.1351) (width 0.35) (layer B.Cu) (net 4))
 (segment (start 145.923 70.485) (end 145.923 70.81) (width 0.35) (layer B.Cu) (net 4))
 (segment (start 156.845 63.5) (end 156.845 64.9751) (width 0.35) (layer F.Cu) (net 4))
 (segment (start 156.845 64.9751) (end 157.043 65.1731) (width 0.35) (layer F.Cu) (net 4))
 (segment (start 157.043 65.1731) (end 157.043 72.898) (width 0.35) (layer F.Cu) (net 4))
 (segment (start 145.669 63.5) (end 145.669 67.8186) (width 0.35) (layer F.Cu) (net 4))
 (segment (start 145.669 67.8186) (end 146.7935 68.9431) (width 0.35) (layer F.Cu) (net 4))
 (segment (start 146.7935 68.9431) (end 146.7935 72.4904) (width 0.35) (layer F.Cu) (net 4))
 (segment (start 146.7935 72.4904) (end 148.516 74.2129) (width 0.35) (layer F.Cu) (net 4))
 (segment (start 152.207 80.7872) (end 152.207 80.0121) (width 0.35) (layer B.Cu) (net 4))
 (segment (start 152.207 80.0121) (end 152.273 79.9461) (width 0.35) (layer B.Cu) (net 4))
 (segment (start 152.273 79.9461) (end 152.273 78.994) (width 0.35) (layer B.Cu) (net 4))
 (segment (start 155.829 96.139) (end 156.3223 96.6323) (width 0.35) (layer B.Cu) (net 4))
 (segment (start 156.3223 96.6323) (end 156.3223 101.0282) (width 0.35) (layer B.Cu) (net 4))
 (segment (start 156.3223 101.0282) (end 153.7244 103.6261) (width 0.35) (layer B.Cu) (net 4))
 (segment (start 153.7244 103.6261) (end 149.987 103.6261) (width 0.35) (layer B.Cu) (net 4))
 (segment (start 149.987 102.235) (end 149.987 103.6261) (width 0.35) (layer B.Cu) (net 4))
 (segment (start 156.771 75.438) (end 156.771 74.2129) (width 0.35) (layer F.Cu) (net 4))
 (segment (start 156.771 74.2129) (end 157.043 73.9409) (width 0.35) (layer F.Cu) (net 4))
 (segment (start 157.043 73.9409) (end 157.043 72.898) (width 0.35) (layer F.Cu) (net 4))
 (segment (start 148.516 75.438) (end 148.516 74.2129) (width 0.35) (layer F.Cu) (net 4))
 (segment (start 148.516 74.2129) (end 148.915 73.8139) (width 0.35) (layer F.Cu) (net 4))
 (segment (start 148.915 73.8139) (end 148.915 72.898) (width 0.35) (layer F.Cu) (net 4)))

